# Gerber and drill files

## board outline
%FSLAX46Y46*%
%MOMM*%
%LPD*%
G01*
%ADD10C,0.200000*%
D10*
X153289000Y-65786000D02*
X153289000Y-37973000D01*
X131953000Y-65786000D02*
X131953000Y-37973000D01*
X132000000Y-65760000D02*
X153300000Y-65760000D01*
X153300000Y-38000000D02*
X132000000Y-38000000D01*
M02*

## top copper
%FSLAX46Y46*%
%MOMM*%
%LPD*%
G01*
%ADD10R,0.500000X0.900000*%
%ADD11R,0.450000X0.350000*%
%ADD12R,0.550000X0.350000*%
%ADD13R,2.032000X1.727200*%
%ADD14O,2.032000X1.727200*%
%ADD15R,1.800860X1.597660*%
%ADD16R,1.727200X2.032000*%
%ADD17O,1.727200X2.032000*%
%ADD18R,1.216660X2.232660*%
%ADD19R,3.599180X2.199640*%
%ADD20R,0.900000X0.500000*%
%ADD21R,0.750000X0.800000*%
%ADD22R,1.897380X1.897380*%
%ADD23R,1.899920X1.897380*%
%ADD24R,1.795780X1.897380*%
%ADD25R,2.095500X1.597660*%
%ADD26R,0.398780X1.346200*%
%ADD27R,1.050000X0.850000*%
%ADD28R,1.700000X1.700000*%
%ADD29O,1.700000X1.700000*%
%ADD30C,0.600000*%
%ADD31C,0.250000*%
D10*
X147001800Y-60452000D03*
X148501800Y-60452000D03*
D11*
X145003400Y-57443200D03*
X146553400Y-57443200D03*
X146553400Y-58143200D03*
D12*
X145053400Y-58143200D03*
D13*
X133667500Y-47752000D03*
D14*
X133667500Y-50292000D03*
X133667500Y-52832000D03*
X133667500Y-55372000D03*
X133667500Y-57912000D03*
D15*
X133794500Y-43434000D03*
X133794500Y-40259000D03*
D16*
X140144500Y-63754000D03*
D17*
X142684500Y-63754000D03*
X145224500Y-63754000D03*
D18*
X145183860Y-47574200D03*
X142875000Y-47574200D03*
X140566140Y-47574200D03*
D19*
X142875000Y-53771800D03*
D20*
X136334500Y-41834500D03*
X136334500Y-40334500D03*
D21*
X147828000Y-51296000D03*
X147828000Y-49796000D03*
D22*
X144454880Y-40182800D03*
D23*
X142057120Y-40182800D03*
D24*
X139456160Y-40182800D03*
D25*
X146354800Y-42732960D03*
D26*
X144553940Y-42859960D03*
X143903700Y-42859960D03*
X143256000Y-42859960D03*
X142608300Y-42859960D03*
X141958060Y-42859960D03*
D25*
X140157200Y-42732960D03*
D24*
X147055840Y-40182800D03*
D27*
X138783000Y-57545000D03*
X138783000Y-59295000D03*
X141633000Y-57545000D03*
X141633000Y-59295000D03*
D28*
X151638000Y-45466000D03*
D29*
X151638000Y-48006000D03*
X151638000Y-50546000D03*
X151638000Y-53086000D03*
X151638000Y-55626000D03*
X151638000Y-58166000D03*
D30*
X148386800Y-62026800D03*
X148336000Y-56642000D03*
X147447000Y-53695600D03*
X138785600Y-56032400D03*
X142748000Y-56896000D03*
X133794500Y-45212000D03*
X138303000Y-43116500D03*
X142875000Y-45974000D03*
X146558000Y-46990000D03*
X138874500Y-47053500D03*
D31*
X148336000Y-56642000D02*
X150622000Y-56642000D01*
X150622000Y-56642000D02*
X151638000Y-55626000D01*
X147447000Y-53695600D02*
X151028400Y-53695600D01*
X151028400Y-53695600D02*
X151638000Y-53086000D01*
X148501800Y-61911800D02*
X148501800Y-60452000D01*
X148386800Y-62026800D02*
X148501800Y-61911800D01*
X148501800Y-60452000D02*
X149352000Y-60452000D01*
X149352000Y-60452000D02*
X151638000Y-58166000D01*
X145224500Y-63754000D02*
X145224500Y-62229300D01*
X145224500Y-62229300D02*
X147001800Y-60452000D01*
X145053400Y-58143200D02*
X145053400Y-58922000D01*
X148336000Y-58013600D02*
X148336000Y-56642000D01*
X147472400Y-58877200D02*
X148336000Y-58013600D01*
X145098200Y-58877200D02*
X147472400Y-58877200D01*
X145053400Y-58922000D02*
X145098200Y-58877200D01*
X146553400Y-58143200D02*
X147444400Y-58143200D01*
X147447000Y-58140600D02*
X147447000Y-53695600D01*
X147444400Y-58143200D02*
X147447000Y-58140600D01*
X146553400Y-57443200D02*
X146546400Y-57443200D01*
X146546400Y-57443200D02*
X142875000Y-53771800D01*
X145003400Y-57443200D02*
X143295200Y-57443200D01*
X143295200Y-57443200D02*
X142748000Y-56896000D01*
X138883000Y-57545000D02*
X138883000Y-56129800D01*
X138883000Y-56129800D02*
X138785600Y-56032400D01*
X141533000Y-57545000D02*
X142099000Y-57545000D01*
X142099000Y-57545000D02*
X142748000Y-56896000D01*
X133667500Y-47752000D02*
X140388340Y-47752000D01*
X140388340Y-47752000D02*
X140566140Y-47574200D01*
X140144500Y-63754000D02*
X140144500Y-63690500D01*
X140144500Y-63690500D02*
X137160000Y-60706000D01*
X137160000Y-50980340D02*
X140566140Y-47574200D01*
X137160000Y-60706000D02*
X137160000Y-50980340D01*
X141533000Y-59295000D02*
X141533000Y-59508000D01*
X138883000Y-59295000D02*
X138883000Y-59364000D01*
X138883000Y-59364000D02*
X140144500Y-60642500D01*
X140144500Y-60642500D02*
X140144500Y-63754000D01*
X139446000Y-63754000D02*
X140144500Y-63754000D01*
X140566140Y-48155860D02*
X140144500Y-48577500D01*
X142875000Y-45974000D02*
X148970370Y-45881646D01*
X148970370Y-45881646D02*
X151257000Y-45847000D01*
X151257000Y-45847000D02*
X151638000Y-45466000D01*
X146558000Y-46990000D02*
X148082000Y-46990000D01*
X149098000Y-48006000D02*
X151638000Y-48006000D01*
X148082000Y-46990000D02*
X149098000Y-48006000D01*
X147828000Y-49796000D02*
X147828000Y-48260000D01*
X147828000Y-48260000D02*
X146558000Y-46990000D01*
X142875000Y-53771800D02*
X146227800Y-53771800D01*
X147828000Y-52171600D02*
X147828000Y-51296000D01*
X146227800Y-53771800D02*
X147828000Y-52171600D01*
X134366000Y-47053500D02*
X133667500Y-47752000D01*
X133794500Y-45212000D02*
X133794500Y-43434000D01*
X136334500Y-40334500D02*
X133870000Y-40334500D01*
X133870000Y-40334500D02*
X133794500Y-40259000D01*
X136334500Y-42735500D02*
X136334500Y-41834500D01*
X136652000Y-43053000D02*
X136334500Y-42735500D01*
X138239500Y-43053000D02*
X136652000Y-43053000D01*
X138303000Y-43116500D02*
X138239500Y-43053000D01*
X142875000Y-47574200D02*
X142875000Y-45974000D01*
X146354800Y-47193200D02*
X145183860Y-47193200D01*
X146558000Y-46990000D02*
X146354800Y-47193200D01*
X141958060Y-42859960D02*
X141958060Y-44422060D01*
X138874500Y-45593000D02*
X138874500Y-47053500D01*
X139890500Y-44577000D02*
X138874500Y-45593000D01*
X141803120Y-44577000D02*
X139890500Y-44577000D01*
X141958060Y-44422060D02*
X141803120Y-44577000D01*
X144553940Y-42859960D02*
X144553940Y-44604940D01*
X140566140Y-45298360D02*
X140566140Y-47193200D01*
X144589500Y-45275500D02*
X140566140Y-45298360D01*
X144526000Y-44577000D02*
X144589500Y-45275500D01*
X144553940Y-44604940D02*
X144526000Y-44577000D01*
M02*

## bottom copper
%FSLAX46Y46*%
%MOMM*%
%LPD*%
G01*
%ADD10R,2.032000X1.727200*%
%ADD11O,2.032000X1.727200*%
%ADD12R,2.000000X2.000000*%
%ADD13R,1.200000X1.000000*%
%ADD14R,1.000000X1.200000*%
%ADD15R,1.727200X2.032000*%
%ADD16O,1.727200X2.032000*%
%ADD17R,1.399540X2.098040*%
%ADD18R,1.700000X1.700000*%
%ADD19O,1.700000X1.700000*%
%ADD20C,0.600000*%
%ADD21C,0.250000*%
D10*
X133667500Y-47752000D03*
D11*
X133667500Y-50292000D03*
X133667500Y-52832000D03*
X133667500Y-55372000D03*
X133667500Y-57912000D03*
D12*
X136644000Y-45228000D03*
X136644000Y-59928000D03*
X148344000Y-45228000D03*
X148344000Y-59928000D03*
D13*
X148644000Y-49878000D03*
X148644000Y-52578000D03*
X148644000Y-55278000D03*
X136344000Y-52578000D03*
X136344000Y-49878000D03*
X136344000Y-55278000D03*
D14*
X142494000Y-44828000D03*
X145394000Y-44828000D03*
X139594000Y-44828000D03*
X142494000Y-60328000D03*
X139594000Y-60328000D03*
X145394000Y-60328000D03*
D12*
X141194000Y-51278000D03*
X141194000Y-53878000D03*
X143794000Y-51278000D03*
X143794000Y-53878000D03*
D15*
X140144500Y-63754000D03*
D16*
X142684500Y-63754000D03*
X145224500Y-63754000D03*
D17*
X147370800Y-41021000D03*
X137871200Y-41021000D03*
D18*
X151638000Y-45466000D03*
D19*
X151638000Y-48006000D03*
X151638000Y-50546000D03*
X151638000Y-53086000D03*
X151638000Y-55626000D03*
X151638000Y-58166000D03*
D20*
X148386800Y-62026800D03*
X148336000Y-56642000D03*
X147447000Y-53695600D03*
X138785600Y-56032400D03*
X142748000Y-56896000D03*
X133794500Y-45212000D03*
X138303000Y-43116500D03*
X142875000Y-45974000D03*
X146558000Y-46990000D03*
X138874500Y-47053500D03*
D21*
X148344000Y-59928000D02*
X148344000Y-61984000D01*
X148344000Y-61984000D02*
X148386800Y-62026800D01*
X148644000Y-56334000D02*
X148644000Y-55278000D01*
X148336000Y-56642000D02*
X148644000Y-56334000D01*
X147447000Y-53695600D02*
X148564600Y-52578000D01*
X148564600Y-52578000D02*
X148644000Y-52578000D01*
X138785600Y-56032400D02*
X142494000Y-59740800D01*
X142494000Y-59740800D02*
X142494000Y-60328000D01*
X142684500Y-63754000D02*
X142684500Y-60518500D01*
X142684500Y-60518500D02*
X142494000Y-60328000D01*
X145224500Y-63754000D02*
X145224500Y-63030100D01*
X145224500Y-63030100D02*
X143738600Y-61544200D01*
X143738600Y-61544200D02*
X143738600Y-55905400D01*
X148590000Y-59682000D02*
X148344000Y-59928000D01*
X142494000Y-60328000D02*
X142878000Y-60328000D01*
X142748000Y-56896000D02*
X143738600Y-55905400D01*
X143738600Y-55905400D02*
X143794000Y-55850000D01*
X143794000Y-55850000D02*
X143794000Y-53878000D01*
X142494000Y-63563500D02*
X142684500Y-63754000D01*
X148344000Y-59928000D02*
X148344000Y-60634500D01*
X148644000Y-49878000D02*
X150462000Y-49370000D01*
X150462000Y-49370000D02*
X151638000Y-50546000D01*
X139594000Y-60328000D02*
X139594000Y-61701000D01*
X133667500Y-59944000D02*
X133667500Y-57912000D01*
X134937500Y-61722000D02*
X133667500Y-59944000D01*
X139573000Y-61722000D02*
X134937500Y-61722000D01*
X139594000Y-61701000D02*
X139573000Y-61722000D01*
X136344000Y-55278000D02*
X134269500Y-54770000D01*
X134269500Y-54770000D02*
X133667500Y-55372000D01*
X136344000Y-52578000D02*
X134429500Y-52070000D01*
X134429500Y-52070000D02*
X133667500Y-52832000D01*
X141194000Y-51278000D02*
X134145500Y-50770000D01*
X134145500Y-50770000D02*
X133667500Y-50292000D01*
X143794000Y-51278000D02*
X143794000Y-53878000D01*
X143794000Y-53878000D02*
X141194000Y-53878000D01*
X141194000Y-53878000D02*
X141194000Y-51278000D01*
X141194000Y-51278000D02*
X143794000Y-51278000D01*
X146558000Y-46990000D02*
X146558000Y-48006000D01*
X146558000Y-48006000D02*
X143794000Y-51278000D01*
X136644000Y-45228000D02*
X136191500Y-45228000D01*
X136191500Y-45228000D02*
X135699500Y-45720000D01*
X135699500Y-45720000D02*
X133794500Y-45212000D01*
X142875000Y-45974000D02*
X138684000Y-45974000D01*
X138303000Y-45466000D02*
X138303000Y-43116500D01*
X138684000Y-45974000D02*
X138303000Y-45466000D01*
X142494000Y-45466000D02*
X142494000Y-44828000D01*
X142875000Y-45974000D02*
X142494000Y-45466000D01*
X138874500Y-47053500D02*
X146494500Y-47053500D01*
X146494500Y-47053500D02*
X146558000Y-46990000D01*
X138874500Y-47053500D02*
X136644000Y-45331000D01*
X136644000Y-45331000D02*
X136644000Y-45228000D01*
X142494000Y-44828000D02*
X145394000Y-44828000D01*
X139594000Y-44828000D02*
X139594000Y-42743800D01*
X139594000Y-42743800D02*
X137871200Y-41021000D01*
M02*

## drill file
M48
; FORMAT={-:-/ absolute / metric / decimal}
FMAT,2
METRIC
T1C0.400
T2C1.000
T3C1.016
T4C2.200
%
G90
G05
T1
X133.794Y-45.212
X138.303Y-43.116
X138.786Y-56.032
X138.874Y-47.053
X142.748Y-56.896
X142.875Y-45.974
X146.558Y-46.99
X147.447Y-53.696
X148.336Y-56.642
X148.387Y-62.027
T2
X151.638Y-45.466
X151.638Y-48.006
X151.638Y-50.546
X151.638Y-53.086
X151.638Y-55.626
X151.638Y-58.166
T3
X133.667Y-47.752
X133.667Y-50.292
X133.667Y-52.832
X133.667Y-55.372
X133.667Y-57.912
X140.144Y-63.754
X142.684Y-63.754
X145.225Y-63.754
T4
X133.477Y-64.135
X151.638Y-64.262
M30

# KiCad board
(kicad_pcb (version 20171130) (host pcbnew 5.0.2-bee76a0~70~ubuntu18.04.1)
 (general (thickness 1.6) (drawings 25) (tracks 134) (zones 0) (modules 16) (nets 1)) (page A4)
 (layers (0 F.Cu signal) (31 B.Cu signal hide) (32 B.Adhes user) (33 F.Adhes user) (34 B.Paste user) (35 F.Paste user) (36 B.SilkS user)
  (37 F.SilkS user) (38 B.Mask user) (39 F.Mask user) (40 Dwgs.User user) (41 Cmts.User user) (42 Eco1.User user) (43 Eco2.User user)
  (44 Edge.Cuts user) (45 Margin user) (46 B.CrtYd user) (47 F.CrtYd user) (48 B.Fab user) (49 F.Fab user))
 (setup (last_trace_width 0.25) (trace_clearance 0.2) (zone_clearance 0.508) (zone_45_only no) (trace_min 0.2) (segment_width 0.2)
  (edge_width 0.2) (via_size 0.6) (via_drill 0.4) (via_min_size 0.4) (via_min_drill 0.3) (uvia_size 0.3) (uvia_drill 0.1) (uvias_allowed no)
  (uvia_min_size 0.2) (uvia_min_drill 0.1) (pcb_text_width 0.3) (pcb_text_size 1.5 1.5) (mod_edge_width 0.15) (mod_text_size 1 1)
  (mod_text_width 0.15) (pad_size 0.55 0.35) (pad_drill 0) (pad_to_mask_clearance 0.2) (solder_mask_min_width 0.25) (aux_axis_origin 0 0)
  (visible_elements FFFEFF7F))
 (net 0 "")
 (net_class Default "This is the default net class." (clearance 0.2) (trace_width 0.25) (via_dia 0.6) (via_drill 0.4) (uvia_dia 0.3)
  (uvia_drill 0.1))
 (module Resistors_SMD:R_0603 (layer F.Cu) (at 147.7518 60.452)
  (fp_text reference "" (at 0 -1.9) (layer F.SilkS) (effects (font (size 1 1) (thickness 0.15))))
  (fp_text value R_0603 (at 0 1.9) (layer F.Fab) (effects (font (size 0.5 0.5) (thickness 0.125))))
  (pad 1 smd rect (at -0.75 0) (size 0.5 0.9) (layers F.Cu F.Paste F.Mask))
  (pad 2 smd rect (at 0.75 0) (size 0.5 0.9) (layers F.Cu F.Paste F.Mask)))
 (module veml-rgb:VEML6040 (layer F.Cu) (at 145.9484 56.7182)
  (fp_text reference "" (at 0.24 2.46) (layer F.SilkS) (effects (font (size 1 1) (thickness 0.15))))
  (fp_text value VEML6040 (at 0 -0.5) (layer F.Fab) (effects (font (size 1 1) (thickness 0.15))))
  (pad GND smd rect (at -0.945 0.725) (size 0.45 0.35) (layers F.Cu F.Paste F.Mask))
  (pad +V smd rect (at 0.605 0.725) (size 0.45 0.35) (layers F.Cu F.Paste F.Mask))
  (pad 3 smd rect (at 0.605 1.425) (size 0.45 0.35) (layers F.Cu F.Paste F.Mask))
  (pad 2 smd rect (at -0.895 1.425) (size 0.55 0.35) (layers F.Cu F.Paste F.Mask)))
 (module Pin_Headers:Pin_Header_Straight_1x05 (layer F.Cu) (at 133.6675 47.752)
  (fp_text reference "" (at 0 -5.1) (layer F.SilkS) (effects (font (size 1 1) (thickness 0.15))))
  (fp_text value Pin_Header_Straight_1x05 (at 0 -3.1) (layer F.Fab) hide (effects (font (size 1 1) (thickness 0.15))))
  (pad 1 thru_hole rect (at 0 0) (size 2.032 1.7272) (drill 1.016) (layers *.Cu *.Mask F.SilkS))
  (pad 2 thru_hole oval (at 0 2.54) (size 2.032 1.7272) (drill 1.016) (layers *.Cu *.Mask F.SilkS))
  (pad 3 thru_hole oval (at 0 5.08) (size 2.032 1.7272) (drill 1.016) (layers *.Cu *.Mask F.SilkS))
  (pad 4 thru_hole oval (at 0 7.62) (size 2.032 1.7272) (drill 1.016) (layers *.Cu *.Mask F.SilkS))
  (pad 5 thru_hole oval (at 0 10.16) (size 2.032 1.7272) (drill 1.016) (layers *.Cu *.Mask F.SilkS)))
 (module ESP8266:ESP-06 (layer B.Cu) (at 142.494 52.578 270)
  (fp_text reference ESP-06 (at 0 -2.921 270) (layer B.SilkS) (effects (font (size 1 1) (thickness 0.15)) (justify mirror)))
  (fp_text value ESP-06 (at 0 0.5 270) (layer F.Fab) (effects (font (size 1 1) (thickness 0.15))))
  (pad GND smd rect (at -7.35 5.85 270) (size 2 2) (layers B.Cu B.Paste B.Mask))
  (pad GP5 smd rect (at 7.35 5.85 270) (size 2 2) (layers B.Cu B.Paste B.Mask))
  (pad GP16 smd rect (at -7.35 -5.85 270) (size 2 2) (layers B.Cu B.Paste B.Mask))
  (pad GP15 smd rect (at 7.35 -5.85 270) (size 2 2) (layers B.Cu B.Paste B.Mask))
  (pad GP14 smd rect (at -2.7 -6.15 270) (size 1 1.2) (layers B.Cu B.Paste B.Mask))
  (pad GP12 smd rect (at 0 -6.15 270) (size 1 1.2) (layers B.Cu B.Paste B.Mask))
  (pad GP13 smd rect (at 2.7 -6.15 270) (size 1 1.2) (layers B.Cu B.Paste B.Mask))
  (pad TX smd rect (at 0 6.15 270) (size 1 1.2) (layers B.Cu B.Paste B.Mask))
  (pad RST smd rect (at -2.7 6.15 270) (size 1 1.2) (layers B.Cu B.Paste B.Mask))
  (pad RX smd rect (at 2.7 6.15 270) (size 1 1.2) (layers B.Cu B.Paste B.Mask))
  (pad 3.3 smd rect (at -7.75 0 270) (size 1.2 1) (layers B.Cu B.Paste B.Mask))
  (pad CHPD smd rect (at -7.75 -2.9 270) (size 1.2 1) (layers B.Cu B.Paste B.Mask))
  (pad ANT smd rect (at -7.75 2.9 270) (size 1.2 1) (layers B.Cu B.Paste B.Mask))
  (pad GP2 smd rect (at 7.75 0 270) (size 1.2 1) (layers B.Cu B.Paste B.Mask))
  (pad GP0 smd rect (at 7.75 2.9 270) (size 1.2 1) (layers B.Cu B.Paste B.Mask))
  (pad GP4 smd rect (at 7.75 -2.9 270) (size 1.2 1) (layers B.Cu B.Paste B.Mask))
  (pad GND smd rect (at -1.3 1.3 270) (size 2 2) (layers B.Cu B.Paste B.Mask))
  (pad GND smd rect (at 1.3 1.3 270) (size 2 2) (layers B.Cu B.Paste B.Mask))
  (pad GND smd rect (at -1.3 -1.3 270) (size 2 2) (layers B.Cu B.Paste B.Mask))
  (pad GND smd rect (at 1.3 -1.3 270) (size 2 2) (layers B.Cu B.Paste B.Mask)))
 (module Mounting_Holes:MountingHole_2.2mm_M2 (layer F.Cu) (at 133.477 64.135)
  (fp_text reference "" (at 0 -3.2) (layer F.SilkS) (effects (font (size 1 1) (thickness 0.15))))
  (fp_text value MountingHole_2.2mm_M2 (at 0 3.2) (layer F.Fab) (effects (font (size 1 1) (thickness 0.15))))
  (pad 1 np_thru_hole circle (at 0 0) (size 2.2 2.2) (drill 2.2) (layers *.Cu *.Mask F.SilkS)))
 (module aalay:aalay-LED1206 (layer F.Cu) (at 133.7945 41.8465 90)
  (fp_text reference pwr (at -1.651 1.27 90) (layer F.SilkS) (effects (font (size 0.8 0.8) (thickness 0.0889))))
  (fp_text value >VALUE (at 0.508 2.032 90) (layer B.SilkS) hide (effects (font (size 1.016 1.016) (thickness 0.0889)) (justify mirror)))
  (pad A smd rect (at -1.5875 0 90) (size 1.59766 1.80086) (layers F.Cu F.Paste F.Mask))
  (pad K smd rect (at 1.5875 0 90) (size 1.59766 1.80086) (layers F.Cu F.Paste F.Mask)))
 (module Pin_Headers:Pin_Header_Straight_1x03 (layer F.Cu) (at 140.1445 63.754 90)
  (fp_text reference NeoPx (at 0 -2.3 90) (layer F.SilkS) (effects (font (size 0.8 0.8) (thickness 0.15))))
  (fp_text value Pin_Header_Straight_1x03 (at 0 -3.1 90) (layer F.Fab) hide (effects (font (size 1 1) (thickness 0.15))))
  (pad 1 thru_hole rect (at 0 0 90) (size 2.032 1.7272) (drill 1.016) (layers *.Cu *.Mask F.SilkS))
  (pad 2 thru_hole oval (at 0 2.54 90) (size 2.032 1.7272) (drill 1.016) (layers *.Cu *.Mask F.SilkS))
  (pad 3 thru_hole oval (at 0 5.08 90) (size 2.032 1.7272) (drill 1.016) (layers *.Cu *.Mask F.SilkS)))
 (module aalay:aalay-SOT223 (layer F.Cu) (at 142.875 50.673 180)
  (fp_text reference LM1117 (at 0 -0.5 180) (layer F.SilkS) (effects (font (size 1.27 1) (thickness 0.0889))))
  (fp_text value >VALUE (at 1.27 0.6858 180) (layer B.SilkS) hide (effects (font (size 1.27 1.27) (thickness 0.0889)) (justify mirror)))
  (pad GND smd rect (at -2.30886 3.0988 180) (size 1.21666 2.23266) (layers F.Cu F.Paste F.Mask))
  (pad OUT smd rect (at 0 3.0988 180) (size 1.21666 2.23266) (layers F.Cu F.Paste F.Mask))
  (pad IN smd rect (at 2.30886 3.0988 180) (size 1.21666 2.23266) (layers F.Cu F.Paste F.Mask))
  (pad OUT smd rect (at 0 -3.0988 180) (size 3.59918 2.19964) (layers F.Cu F.Paste F.Mask)))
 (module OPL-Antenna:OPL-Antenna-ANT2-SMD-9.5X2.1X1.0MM (layer B.Cu) (at 142.621 41.021 180)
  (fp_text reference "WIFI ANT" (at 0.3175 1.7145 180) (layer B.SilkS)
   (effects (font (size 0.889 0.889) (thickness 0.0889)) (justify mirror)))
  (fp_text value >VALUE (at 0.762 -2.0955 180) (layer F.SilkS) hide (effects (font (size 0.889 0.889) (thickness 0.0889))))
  (pad 1 smd rect (at -4.7498 0 180) (size 1.39954 2.09804) (layers B.Cu B.Paste B.Mask))
  (pad 2 smd rect (at 4.7498 0 180) (size 1.39954 2.09804) (layers B.Cu B.Paste B.Mask)))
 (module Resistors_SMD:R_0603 (layer F.Cu) (at 136.3345 41.0845 90)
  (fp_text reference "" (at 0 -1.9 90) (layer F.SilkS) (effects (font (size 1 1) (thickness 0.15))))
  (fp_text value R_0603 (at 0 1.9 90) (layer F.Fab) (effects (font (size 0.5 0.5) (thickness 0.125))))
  (pad 1 smd rect (at -0.75 0 90) (size 0.5 0.9) (layers F.Cu F.Paste F.Mask))
  (pad 2 smd rect (at 0.75 0 90) (size 0.5 0.9) (layers F.Cu F.Paste F.Mask)))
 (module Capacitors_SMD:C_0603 (layer F.Cu) (at 147.828 50.546 90)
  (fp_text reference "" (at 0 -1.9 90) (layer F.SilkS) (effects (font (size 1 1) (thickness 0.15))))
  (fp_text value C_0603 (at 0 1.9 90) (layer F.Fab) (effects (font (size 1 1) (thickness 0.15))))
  (pad 1 smd rect (at -0.75 0 90) (size 0.8 0.75) (layers F.Cu F.Paste F.Mask))
  (pad 2 smd rect (at 0.75 0 90) (size 0.8 0.75) (layers F.Cu F.Paste F.Mask)))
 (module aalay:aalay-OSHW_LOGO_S (layer F.Cu) (at 150.622 39.878)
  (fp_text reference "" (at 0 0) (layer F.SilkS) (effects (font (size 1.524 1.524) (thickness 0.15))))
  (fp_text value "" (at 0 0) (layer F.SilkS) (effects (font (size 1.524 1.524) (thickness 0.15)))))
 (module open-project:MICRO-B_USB (layer F.Cu) (at 143.256 38.735 180)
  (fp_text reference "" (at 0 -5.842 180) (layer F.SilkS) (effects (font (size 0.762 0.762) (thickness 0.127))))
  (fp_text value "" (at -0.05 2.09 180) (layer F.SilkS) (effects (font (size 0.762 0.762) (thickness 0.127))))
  (pad "" smd rect (at -1.19888 -1.4478 180) (size 1.89738 1.89738) (layers F.Cu F.Paste F.Mask))
  (pad "" smd rect (at 1.19888 -1.4478 180) (size 1.89992 1.89738) (layers F.Cu F.Paste F.Mask))
  (pad "" smd rect (at 3.79984 -1.4478 180) (size 1.79578 1.89738) (layers F.Cu F.Paste F.Mask))
  (pad "" smd rect (at -3.0988 -3.99796 180) (size 2.0955 1.59766) (layers F.Cu F.Paste F.Mask))
  (pad +5 smd rect (at -1.29794 -4.12496 180) (size 0.39878 1.3462) (layers F.Cu F.Paste F.Mask) (clearance 0.2032))
  (pad 2 smd rect (at -0.6477 -4.12496 180) (size 0.39878 1.3462) (layers F.Cu F.Paste F.Mask) (clearance 0.2032))
  (pad 3 smd rect (at 0 -4.12496 180) (size 0.39878 1.3462) (layers F.Cu F.Paste F.Mask) (clearance 0.2032))
  (pad 4 smd rect (at 0.6477 -4.12496 180) (size 0.39878 1.3462) (layers F.Cu F.Paste F.Mask) (clearance 0.2032))
  (pad GND smd rect (at 1.29794 -4.12496 180) (size 0.39878 1.3462) (layers F.Cu F.Paste F.Mask) (clearance 0.2032))
  (pad "" smd rect (at 3.0988 -3.99796 180) (size 2.0955 1.59766) (layers F.Cu F.Paste F.Mask))
  (pad "" smd rect (at -3.79984 -1.4478 180) (size 1.79578 1.89738) (layers F.Cu F.Paste F.Mask)))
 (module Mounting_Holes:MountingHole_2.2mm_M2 (layer F.Cu) (at 151.638 64.262)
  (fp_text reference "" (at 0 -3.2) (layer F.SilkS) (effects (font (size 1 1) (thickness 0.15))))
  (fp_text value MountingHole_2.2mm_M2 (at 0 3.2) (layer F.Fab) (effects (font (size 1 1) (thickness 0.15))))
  (pad 1 np_thru_hole circle (at 0 0) (size 2.2 2.2) (drill 2.2) (layers *.Cu *.Mask F.SilkS)))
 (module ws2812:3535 (layer F.Cu) (at 140.208 58.42 180)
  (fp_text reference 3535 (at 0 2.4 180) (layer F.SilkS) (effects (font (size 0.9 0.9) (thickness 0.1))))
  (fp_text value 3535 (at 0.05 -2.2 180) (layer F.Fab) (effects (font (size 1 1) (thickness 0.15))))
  (pad IN smd rect (at 1.325 0.875 180) (size 1.05 0.85) (drill (offset 0.1 0)) (layers F.Cu F.Paste F.Mask))
  (pad VDD smd rect (at 1.325 -0.875 180) (size 1.05 0.85) (drill (offset 0.1 0)) (layers F.Cu F.Paste F.Mask))
  (pad GND smd rect (at -1.325 0.875 180) (size 1.05 0.85) (drill (offset -0.1 0)) (layers F.Cu F.Paste F.Mask))
  (pad OUT smd rect (at -1.325 -0.875 180) (size 1.05 0.85) (drill (offset -0.1 0)) (layers F.Cu F.Paste F.Mask)))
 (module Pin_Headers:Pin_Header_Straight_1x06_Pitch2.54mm (layer F.Cu) (at 151.638 45.466)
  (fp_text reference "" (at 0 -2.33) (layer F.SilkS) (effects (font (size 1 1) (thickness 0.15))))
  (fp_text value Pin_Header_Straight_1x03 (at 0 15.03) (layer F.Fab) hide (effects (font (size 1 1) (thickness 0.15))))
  (pad 1 thru_hole rect (at 0 0) (size 1.7 1.7) (drill 1) (layers *.Cu *.Mask))
  (pad 2 thru_hole oval (at 0 2.54) (size 1.7 1.7) (drill 1) (layers *.Cu *.Mask))
  (pad 3 thru_hole oval (at 0 5.08) (size 1.7 1.7) (drill 1) (layers *.Cu *.Mask))
  (pad 4 thru_hole oval (at 0 7.62) (size 1.7 1.7) (drill 1) (layers *.Cu *.Mask))
  (pad 5 thru_hole oval (at 0 10.16) (size 1.7 1.7) (drill 1) (layers *.Cu *.Mask))
  (pad 6 thru_hole oval (at 0 12.7) (size 1.7 1.7) (drill 1) (layers *.Cu *.Mask)))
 (gr_line (start 153.289 65.786) (end 153.289 37.973) (angle 90) (layer Edge.Cuts) (width 0.2))
 (gr_line (start 131.953 65.786) (end 131.953 37.973) (angle 90) (layer Edge.Cuts) (width 0.2))
 (gr_line (start 132 65.76) (end 153.3 65.76) (angle 90) (layer Edge.Cuts) (width 0.2))
 (gr_line (start 153.3 38) (end 132 38) (angle 90) (layer Edge.Cuts) (width 0.2))
 (segment (start 148.336 56.642) (end 150.622 56.642) (width 0.25) (layer F.Cu) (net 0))
 (segment (start 150.622 56.642) (end 151.638 55.626) (width 0.25) (layer F.Cu) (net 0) (status 800000))
 (segment (start 147.447 53.6956) (end 151.0284 53.6956) (width 0.25) (layer F.Cu) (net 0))
 (segment (start 151.0284 53.6956) (end 151.638 53.086) (width 0.25) (layer F.Cu) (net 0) (status 800000))
 (segment (start 148.344 59.928) (end 148.344 61.984) (width 0.25) (layer B.Cu) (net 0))
 (segment (start 148.5018 61.9118) (end 148.5018 60.452) (width 0.25) (layer F.Cu) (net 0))
 (segment (start 148.3868 62.0268) (end 148.5018 61.9118) (width 0.25) (layer F.Cu) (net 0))
 (via (at 148.3868 62.0268) (size 0.6) (drill 0.4) (layers F.Cu B.Cu) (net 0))
 (segment (start 148.344 61.984) (end 148.3868 62.0268) (width 0.25) (layer B.Cu) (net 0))
 (segment (start 148.5018 60.452) (end 149.352 60.452) (width 0.25) (layer F.Cu) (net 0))
 (segment (start 149.352 60.452) (end 151.638 58.166) (width 0.25) (layer F.Cu) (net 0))
 (segment (start 145.2245 63.754) (end 145.2245 62.2293) (width 0.25) (layer F.Cu) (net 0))
 (segment (start 145.2245 62.2293) (end 147.0018 60.452) (width 0.25) (layer F.Cu) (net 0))
 (segment (start 145.0534 58.1432) (end 145.0534 58.922) (width 0.25) (layer F.Cu) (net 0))
 (segment (start 148.644 56.334) (end 148.644 55.278) (width 0.25) (layer B.Cu) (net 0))
 (segment (start 148.336 56.642) (end 148.644 56.334) (width 0.25) (layer B.Cu) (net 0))
 (via (at 148.336 56.642) (size 0.6) (drill 0.4) (layers F.Cu B.Cu) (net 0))
 (segment (start 148.336 58.0136) (end 148.336 56.642) (width 0.25) (layer F.Cu) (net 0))
 (segment (start 147.4724 58.8772) (end 148.336 58.0136) (width 0.25) (layer F.Cu) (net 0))
 (segment (start 145.0982 58.8772) (end 147.4724 58.8772) (width 0.25) (layer F.Cu) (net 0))
 (segment (start 145.0534 58.922) (end 145.0982 58.8772) (width 0.25) (layer F.Cu) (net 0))
 (segment (start 146.5534 58.1432) (end 147.4444 58.1432) (width 0.25) (layer F.Cu) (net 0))
 (segment (start 147.447 53.6956) (end 148.5646 52.578) (width 0.25) (layer B.Cu) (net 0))
 (via (at 147.447 53.6956) (size 0.6) (drill 0.4) (layers F.Cu B.Cu) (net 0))
 (segment (start 147.447 58.1406) (end 147.447 53.6956) (width 0.25) (layer F.Cu) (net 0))
 (segment (start 147.4444 58.1432) (end 147.447 58.1406) (width 0.25) (layer F.Cu) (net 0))
 (segment (start 148.5646 52.578) (end 148.644 52.578) (width 0.25) (layer B.Cu) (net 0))
 (segment (start 146.5534 57.4432) (end 146.5464 57.4432) (width 0.25) (layer F.Cu) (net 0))
 (segment (start 146.5464 57.4432) (end 142.875 53.7718) (width 0.25) (layer F.Cu) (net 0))
 (segment (start 145.0034 57.4432) (end 143.2952 57.4432) (width 0.25) (layer F.Cu) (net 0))
 (segment (start 143.2952 57.4432) (end 142.748 56.896) (width 0.25) (layer F.Cu) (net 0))
 (segment (start 138.883 57.545) (end 138.883 56.1298) (width 0.25) (layer F.Cu) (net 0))
 (segment (start 138.7856 56.0324) (end 142.494 59.7408) (width 0.25) (layer B.Cu) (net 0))
 (via (at 138.7856 56.0324) (size 0.6) (drill 0.4) (layers F.Cu B.Cu) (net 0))
 (segment (start 138.883 56.1298) (end 138.7856 56.0324) (width 0.25) (layer F.Cu) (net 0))
 (segment (start 142.494 59.7408) (end 142.494 60.328) (width 0.25) (layer B.Cu) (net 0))
 (segment (start 142.6845 63.754) (end 142.6845 60.5185) (width 0.25) (layer B.Cu) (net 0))
 (segment (start 142.6845 60.5185) (end 142.494 60.328) (width 0.25) (layer B.Cu) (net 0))
 (segment (start 145.2245 63.754) (end 145.2245 63.0301) (width 0.25) (layer B.Cu) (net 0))
 (segment (start 145.2245 63.0301) (end 143.7386 61.5442) (width 0.25) (layer B.Cu) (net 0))
 (segment (start 143.7386 61.5442) (end 143.7386 55.9054) (width 0.25) (layer B.Cu) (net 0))
 (segment (start 148.59 59.682) (end 148.344 59.928) (width 0.25) (layer B.Cu) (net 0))
 (segment (start 142.494 60.328) (end 142.878 60.328) (width 0.25) (layer B.Cu) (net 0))
 (segment (start 141.533 57.545) (end 142.099 57.545) (width 0.25) (layer F.Cu) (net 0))
 (segment (start 142.099 57.545) (end 142.748 56.896) (width 0.25) (layer F.Cu) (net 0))
 (via (at 142.748 56.896) (size 0.6) (drill 0.4) (layers F.Cu B.Cu) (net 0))
 (segment (start 142.748 56.896) (end 143.7386 55.9054) (width 0.25) (layer B.Cu) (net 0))
 (segment (start 143.7386 55.9054) (end 143.794 55.85) (width 0.25) (layer B.Cu) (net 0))
 (segment (start 143.794 55.85) (end 143.794 53.878) (width 0.25) (layer B.Cu) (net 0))
 (segment (start 133.6675 47.752) (end 140.38834 47.752) (width 0.25) (layer F.Cu) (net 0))
 (segment (start 140.38834 47.752) (end 140.56614 47.5742) (width 0.25) (layer F.Cu) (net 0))
 (segment (start 140.1445 63.754) (end 140.1445 63.6905) (width 0.25) (layer F.Cu) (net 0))
 (segment (start 140.1445 63.6905) (end 137.16 60.706) (width 0.25) (layer F.Cu) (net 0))
 (segment (start 137.16 50.98034) (end 140.56614 47.5742) (width 0.25) (layer F.Cu) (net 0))
 (segment (start 137.16 60.706) (end 137.16 50.98034) (width 0.25) (layer F.Cu) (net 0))
 (segment (start 142.494 63.5635) (end 142.6845 63.754) (width 0.25) (layer B.Cu) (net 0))
 (segment (start 141.533 59.295) (end 141.533 59.508) (width 0.25) (layer F.Cu) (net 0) (status 30))
 (segment (start 138.883 59.295) (end 138.883 59.364) (width 0.25) (layer F.Cu) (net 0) (status 30))
 (segment (start 138.883 59.364) (end 140.1445 60.6425) (width 0.25) (layer F.Cu) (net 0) (status 10))
 (segment (start 140.1445 60.6425) (end 140.1445 63.754) (width 0.25) (layer F.Cu) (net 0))
 (segment (start 139.446 63.754) (end 140.1445 63.754) (width 0.25) (layer F.Cu) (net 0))
 (segment (start 140.56614 48.15586) (end 140.1445 48.5775) (width 0.25) (layer F.Cu) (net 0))
 (segment (start 148.344 59.928) (end 148.344 60.6345) (width 0.25) (layer B.Cu) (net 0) (status 10))
 (segment (start 148.644 49.878) (end 150.462 49.37) (width 0.25) (layer B.Cu) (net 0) (status 10))
 (segment (start 150.462 49.37) (end 151.638 50.546) (width 0.25) (layer B.Cu) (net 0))
 (segment (start 142.875 45.974) (end 148.97037 45.881646) (width 0.25) (layer F.Cu) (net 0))
 (segment (start 148.97037 45.881646) (end 151.257 45.847) (width 0.25) (layer F.Cu) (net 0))
 (segment (start 151.257 45.847) (end 151.638 45.466) (width 0.25) (layer F.Cu) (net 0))
 (segment (start 146.558 46.99) (end 148.082 46.99) (width 0.25) (layer F.Cu) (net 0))
 (segment (start 149.098 48.006) (end 151.638 48.006) (width 0.25) (layer F.Cu) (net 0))
 (segment (start 148.082 46.99) (end 149.098 48.006) (width 0.25) (layer F.Cu) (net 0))
 (segment (start 147.828 49.796) (end 147.828 48.26) (width 0.25) (layer F.Cu) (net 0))
 (segment (start 147.828 48.26) (end 146.558 46.99) (width 0.25) (layer F.Cu) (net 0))
 (segment (start 142.875 53.7718) (end 146.2278 53.7718) (width 0.25) (layer F.Cu) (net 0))
 (segment (start 147.828 52.1716) (end 147.828 51.296) (width 0.25) (layer F.Cu) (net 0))
 (segment (start 146.2278 53.7718) (end 147.828 52.1716) (width 0.25) (layer F.Cu) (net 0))
 (segment (start 139.594 60.328) (end 139.594 61.701) (width 0.25) (layer B.Cu) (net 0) (status 10))
 (segment (start 133.6675 59.944) (end 133.6675 57.912) (width 0.25) (layer B.Cu) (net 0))
 (segment (start 134.9375 61.722) (end 133.6675 59.944) (width 0.25) (layer B.Cu) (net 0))
 (segment (start 139.573 61.722) (end 134.9375 61.722) (width 0.25) (layer B.Cu) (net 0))
 (segment (start 139.594 61.701) (end 139.573 61.722) (width 0.25) (layer B.Cu) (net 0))
 (segment (start 136.344 55.278) (end 134.2695 54.77) (width 0.25) (layer B.Cu) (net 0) (status 10))
 (segment (start 134.2695 54.77) (end 133.6675 55.372) (width 0.25) (layer B.Cu) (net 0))
 (segment (start 136.344 52.578) (end 134.4295 52.07) (width 0.25) (layer B.Cu) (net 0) (status 10))
 (segment (start 134.4295 52.07) (end 133.6675 52.832) (width 0.25) (layer B.Cu) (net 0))
 (segment (start 141.194 51.278) (end 134.1455 50.77) (width 0.25) (layer B.Cu) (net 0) (status 10))
 (segment (start 134.1455 50.77) (end 133.6675 50.292) (width 0.25) (layer B.Cu) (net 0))
 (segment (start 134.366 47.0535) (end 133.6675 47.752) (width 0.25) (layer F.Cu) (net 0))
 (segment (start 143.794 51.278) (end 143.794 53.878) (width 0.25) (layer B.Cu) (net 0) (status 30))
 (segment (start 143.794 53.878) (end 141.194 53.878) (width 0.25) (layer B.Cu) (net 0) (status 30))
 (segment (start 141.194 53.878) (end 141.194 51.278) (width 0.25) (layer B.Cu) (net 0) (status 30))
 (segment (start 141.194 51.278) (end 143.794 51.278) (width 0.25) (layer B.Cu) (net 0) (status 30))
 (segment (start 146.558 46.99) (end 146.558 48.006) (width 0.25) (layer B.Cu) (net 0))
 (segment (start 146.558 48.006) (end 143.794 51.278) (width 0.25) (layer B.Cu) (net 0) (status 20))
 (segment (start 136.644 45.228) (end 136.1915 45.228) (width 0.25) (layer B.Cu) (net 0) (status 30))
 (segment (start 136.1915 45.228) (end 135.6995 45.72) (width 0.25) (layer B.Cu) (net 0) (status 30))
 (segment (start 135.6995 45.72) (end 133.7945 45.212) (width 0.25) (layer B.Cu) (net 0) (status 10))
 (via (at 133.7945 45.212) (size 0.6) (drill 0.4) (layers F.Cu B.Cu) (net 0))
 (segment (start 133.7945 45.212) (end 133.7945 43.434) (width 0.25) (layer F.Cu) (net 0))
 (segment (start 136.3345 40.3345) (end 133.87 40.3345) (width 0.25) (layer F.Cu) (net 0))
 (segment (start 133.87 40.3345) (end 133.7945 40.259) (width 0.25) (layer F.Cu) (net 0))
 (segment (start 142.875 45.974) (end 138.684 45.974) (width 0.25) (layer B.Cu) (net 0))
 (segment (start 136.3345 42.7355) (end 136.3345 41.8345) (width 0.25) (layer F.Cu) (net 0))
 (segment (start 136.652 43.053) (end 136.3345 42.7355) (width 0.25) (layer F.Cu) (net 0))
 (segment (start 138.2395 43.053) (end 136.652 43.053) (width 0.25) (layer F.Cu) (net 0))
 (segment (start 138.303 43.1165) (end 138.2395 43.053) (width 0.25) (layer F.Cu) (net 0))
 (via (at 138.303 43.1165) (size 0.6) (drill 0.4) (layers F.Cu B.Cu) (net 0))
 (segment (start 138.303 45.466) (end 138.303 43.1165) (width 0.25) (layer B.Cu) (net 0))
 (segment (start 138.684 45.974) (end 138.303 45.466) (width 0.25) (layer B.Cu) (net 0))
 (segment (start 142.875 47.5742) (end 142.875 45.974) (width 0.25) (layer F.Cu) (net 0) (status 10))
 (segment (start 142.494 45.466) (end 142.494 44.828) (width 0.25) (layer B.Cu) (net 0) (status 20))
 (segment (start 142.875 45.974) (end 142.494 45.466) (width 0.25) (layer B.Cu) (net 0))
 (via (at 142.875 45.974) (size 0.6) (drill 0.4) (layers F.Cu B.Cu) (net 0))
 (segment (start 138.8745 47.0535) (end 146.4945 47.0535) (width 0.25) (layer B.Cu) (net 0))
 (segment (start 146.3548 47.1932) (end 145.18386 47.1932) (width 0.25) (layer F.Cu) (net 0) (status 20))
 (segment (start 146.558 46.99) (end 146.3548 47.1932) (width 0.25) (layer F.Cu) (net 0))
 (via (at 146.558 46.99) (size 0.6) (drill 0.4) (layers F.Cu B.Cu) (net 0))
 (segment (start 146.4945 47.0535) (end 146.558 46.99) (width 0.25) (layer B.Cu) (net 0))
 (segment (start 141.95806 42.85996) (end 141.95806 44.42206) (width 0.25) (layer F.Cu) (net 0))
 (segment (start 138.8745 47.0535) (end 136.644 45.331) (width 0.25) (layer B.Cu) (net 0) (status 20))
 (via (at 138.8745 47.0535) (size 0.6) (drill 0.4) (layers F.Cu B.Cu) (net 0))
 (segment (start 138.8745 45.593) (end 138.8745 47.0535) (width 0.25) (layer F.Cu) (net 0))
 (segment (start 139.8905 44.577) (end 138.8745 45.593) (width 0.25) (layer F.Cu) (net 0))
 (segment (start 141.80312 44.577) (end 139.8905 44.577) (width 0.25) (layer F.Cu) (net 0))
 (segment (start 141.95806 44.42206) (end 141.80312 44.577) (width 0.25) (layer F.Cu) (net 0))
 (segment (start 136.644 45.331) (end 136.644 45.228) (width 0.25) (layer B.Cu) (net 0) (status 30))
 (segment (start 144.55394 42.85996) (end 144.55394 44.60494) (width 0.25) (layer F.Cu) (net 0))
 (segment (start 140.56614 45.29836) (end 140.56614 47.1932) (width 0.25) (layer F.Cu) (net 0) (status 20))
 (segment (start 144.5895 45.2755) (end 140.56614 45.29836) (width 0.25) (layer F.Cu) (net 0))
 (segment (start 144.526 44.577) (end 144.5895 45.2755) (width 0.25) (layer F.Cu) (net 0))
 (segment (start 144.55394 44.60494) (end 144.526 44.577) (width 0.25) (layer F.Cu) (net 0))
 (segment (start 142.494 44.828) (end 145.394 44.828) (width 0.25) (layer B.Cu) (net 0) (status 30))
 (segment (start 139.594 44.828) (end 139.594 42.7438) (width 0.25) (layer B.Cu) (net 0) (status 10))
 (segment (start 139.594 42.7438) (end 137.8712 41.021) (width 0.25) (layer B.Cu) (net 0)))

